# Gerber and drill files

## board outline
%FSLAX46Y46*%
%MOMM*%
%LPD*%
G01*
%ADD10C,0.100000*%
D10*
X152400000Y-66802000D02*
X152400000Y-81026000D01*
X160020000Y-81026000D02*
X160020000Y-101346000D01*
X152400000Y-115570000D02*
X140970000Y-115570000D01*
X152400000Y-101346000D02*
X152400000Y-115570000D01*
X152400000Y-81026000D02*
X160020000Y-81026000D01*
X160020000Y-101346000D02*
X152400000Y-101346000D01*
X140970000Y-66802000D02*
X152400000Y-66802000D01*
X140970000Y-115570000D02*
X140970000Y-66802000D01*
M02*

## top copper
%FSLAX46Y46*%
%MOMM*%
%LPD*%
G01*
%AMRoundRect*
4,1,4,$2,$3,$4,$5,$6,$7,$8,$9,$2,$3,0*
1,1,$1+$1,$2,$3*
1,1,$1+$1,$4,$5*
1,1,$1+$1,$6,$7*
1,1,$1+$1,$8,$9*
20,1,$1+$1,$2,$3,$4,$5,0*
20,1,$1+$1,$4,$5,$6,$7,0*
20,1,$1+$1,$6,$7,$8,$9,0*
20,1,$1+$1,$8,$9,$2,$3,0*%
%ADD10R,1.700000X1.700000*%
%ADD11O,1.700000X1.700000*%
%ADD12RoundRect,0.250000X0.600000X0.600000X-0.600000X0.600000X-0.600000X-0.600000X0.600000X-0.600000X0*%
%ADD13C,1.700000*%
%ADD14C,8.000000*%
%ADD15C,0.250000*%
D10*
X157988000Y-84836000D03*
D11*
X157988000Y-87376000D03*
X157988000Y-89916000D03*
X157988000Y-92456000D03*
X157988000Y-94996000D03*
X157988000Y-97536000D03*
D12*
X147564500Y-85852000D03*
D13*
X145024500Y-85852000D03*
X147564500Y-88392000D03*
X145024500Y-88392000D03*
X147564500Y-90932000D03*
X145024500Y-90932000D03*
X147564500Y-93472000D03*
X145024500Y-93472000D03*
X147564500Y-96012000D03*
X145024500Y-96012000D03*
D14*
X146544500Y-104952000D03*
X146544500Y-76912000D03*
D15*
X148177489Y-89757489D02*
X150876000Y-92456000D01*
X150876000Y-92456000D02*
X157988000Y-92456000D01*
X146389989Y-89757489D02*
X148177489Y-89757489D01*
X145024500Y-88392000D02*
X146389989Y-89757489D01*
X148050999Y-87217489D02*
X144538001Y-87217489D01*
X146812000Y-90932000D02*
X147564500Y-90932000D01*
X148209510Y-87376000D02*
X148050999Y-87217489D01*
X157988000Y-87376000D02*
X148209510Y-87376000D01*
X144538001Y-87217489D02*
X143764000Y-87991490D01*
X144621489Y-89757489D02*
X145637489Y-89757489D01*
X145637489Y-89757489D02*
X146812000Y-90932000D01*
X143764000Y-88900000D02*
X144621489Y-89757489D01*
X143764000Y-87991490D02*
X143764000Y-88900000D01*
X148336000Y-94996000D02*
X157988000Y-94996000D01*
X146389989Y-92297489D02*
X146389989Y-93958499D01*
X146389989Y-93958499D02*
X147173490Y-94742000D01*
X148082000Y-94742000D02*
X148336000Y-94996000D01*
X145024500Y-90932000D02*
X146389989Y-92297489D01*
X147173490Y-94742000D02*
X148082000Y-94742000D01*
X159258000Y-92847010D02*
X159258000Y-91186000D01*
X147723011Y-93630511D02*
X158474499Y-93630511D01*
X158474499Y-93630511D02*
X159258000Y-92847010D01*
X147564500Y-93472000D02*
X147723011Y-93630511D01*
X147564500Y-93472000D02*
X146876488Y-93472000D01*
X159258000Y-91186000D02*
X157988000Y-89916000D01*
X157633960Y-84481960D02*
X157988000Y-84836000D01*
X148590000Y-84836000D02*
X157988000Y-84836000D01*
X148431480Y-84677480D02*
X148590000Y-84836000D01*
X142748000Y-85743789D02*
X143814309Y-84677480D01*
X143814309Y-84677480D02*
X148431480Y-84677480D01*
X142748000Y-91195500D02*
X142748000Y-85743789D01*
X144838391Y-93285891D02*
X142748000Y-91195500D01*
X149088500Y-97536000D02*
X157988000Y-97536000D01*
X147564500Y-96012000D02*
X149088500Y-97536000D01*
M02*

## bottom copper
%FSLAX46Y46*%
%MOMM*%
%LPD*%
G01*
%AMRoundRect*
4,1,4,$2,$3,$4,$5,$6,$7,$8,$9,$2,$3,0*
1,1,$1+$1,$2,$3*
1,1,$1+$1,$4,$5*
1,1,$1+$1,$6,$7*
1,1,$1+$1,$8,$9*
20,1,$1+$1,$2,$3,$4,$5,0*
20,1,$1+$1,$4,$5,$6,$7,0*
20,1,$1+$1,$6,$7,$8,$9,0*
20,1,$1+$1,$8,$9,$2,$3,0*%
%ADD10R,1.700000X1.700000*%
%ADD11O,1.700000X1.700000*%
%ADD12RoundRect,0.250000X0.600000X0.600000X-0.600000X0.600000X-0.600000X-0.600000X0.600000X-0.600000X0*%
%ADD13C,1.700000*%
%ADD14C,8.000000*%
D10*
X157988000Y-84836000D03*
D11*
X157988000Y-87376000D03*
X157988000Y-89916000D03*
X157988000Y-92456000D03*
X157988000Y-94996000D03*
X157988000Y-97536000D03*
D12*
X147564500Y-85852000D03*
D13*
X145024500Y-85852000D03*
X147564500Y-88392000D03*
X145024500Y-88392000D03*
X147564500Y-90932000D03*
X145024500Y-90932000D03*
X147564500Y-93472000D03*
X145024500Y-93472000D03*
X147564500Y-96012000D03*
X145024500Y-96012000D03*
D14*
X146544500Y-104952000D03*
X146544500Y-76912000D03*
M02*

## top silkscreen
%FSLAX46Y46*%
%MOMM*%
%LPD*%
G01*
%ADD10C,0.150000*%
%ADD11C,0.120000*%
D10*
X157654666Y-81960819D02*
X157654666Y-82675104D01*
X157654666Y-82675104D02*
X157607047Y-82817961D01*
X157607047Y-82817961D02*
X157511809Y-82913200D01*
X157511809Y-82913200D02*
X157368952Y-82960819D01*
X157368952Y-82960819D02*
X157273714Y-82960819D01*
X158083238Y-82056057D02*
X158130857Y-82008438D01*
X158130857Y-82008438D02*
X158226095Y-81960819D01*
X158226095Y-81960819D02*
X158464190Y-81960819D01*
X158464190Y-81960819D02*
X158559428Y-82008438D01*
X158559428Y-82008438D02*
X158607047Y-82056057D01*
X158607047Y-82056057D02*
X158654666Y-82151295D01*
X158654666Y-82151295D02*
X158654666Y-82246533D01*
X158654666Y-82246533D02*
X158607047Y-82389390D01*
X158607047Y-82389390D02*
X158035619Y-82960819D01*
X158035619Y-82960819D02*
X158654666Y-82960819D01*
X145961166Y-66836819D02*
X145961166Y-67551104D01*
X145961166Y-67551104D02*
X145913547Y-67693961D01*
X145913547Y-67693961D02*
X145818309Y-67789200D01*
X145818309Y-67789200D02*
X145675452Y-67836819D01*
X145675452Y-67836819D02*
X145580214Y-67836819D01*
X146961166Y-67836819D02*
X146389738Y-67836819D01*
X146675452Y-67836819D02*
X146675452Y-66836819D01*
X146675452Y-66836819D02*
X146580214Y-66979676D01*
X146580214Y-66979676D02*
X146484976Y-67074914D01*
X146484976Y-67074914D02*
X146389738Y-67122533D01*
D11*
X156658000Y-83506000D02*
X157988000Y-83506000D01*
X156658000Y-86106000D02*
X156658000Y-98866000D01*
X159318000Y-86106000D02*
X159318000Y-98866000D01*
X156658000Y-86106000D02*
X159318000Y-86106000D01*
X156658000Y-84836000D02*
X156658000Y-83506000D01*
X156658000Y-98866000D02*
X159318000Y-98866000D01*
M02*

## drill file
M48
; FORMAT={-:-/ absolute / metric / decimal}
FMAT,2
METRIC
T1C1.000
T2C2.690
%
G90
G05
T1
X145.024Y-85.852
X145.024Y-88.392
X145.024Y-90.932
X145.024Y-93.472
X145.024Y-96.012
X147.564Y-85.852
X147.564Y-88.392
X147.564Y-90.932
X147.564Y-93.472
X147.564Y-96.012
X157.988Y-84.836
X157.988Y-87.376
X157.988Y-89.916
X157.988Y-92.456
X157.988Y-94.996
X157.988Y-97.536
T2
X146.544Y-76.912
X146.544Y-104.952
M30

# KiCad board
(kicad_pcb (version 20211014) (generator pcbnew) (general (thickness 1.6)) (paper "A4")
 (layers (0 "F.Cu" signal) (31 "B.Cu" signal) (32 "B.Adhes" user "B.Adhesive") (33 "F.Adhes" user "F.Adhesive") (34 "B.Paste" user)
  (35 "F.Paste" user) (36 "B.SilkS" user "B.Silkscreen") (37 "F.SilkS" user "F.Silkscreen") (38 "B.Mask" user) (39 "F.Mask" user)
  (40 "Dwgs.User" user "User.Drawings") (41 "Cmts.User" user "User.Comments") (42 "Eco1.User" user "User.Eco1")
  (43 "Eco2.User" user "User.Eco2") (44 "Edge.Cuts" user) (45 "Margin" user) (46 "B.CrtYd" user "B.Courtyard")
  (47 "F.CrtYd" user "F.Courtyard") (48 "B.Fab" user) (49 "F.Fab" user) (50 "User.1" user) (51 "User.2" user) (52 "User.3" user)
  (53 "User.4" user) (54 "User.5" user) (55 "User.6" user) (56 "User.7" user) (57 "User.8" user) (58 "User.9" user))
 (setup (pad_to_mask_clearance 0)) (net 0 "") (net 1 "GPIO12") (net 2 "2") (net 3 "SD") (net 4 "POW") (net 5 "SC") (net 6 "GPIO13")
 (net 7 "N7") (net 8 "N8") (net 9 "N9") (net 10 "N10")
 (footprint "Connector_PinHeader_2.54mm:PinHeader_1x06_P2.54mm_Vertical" (layer "F.Cu") (at 157.988 84.836)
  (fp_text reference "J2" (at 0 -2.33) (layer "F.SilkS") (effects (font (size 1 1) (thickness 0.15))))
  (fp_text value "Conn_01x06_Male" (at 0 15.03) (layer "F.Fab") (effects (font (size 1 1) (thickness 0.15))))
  (fp_line (start -1.33 -1.33) (end 0 -1.33) (layer "F.SilkS") (width 0.12))
  (fp_line (start -1.33 1.27) (end -1.33 14.03) (layer "F.SilkS") (width 0.12))
  (fp_line (start 1.33 1.27) (end 1.33 14.03) (layer "F.SilkS") (width 0.12))
  (fp_line (start -1.33 1.27) (end 1.33 1.27) (layer "F.SilkS") (width 0.12))
  (fp_line (start -1.33 0) (end -1.33 -1.33) (layer "F.SilkS") (width 0.12))
  (fp_line (start -1.33 14.03) (end 1.33 14.03) (layer "F.SilkS") (width 0.12))
  (pad "1" thru_hole rect (at 0 0) (size 1.7 1.7) (drill 1) (layers *.Cu *.Mask) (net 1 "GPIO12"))
  (pad "2" thru_hole oval (at 0 2.54) (size 1.7 1.7) (drill 1) (layers *.Cu *.Mask) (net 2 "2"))
  (pad "3" thru_hole oval (at 0 5.08) (size 1.7 1.7) (drill 1) (layers *.Cu *.Mask) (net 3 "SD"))
  (pad "4" thru_hole oval (at 0 7.62) (size 1.7 1.7) (drill 1) (layers *.Cu *.Mask) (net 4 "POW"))
  (pad "5" thru_hole oval (at 0 10.16) (size 1.7 1.7) (drill 1) (layers *.Cu *.Mask) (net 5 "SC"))
  (pad "6" thru_hole oval (at 0 12.7) (size 1.7 1.7) (drill 1) (layers *.Cu *.Mask) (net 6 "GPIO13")))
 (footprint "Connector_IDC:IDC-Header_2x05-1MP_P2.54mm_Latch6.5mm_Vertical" (layer "B.Cu") (at 147.5645 85.852 180)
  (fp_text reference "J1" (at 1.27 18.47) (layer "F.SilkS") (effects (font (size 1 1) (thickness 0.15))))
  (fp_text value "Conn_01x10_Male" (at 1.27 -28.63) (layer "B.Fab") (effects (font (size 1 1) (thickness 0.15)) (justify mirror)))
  (pad "1" thru_hole roundrect (at 0 0 180) (size 1.7 1.7) (drill 1) (layers *.Cu *.Mask) (roundrect_rratio 0.147059) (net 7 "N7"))
  (pad "2" thru_hole circle (at 2.54 0 180) (size 1.7 1.7) (drill 1) (layers *.Cu *.Mask) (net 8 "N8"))
  (pad "3" thru_hole circle (at 0 -2.54 180) (size 1.7 1.7) (drill 1) (layers *.Cu *.Mask) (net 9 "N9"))
  (pad "4" thru_hole circle (at 2.54 -2.54 180) (size 1.7 1.7) (drill 1) (layers *.Cu *.Mask) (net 4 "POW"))
  (pad "5" thru_hole circle (at 0 -5.08 180) (size 1.7 1.7) (drill 1) (layers *.Cu *.Mask) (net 2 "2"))
  (pad "6" thru_hole circle (at 2.54 -5.08 180) (size 1.7 1.7) (drill 1) (layers *.Cu *.Mask) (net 5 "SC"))
  (pad "7" thru_hole circle (at 0 -7.62 180) (size 1.7 1.7) (drill 1) (layers *.Cu *.Mask) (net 3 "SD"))
  (pad "8" thru_hole circle (at 2.54 -7.62 180) (size 1.7 1.7) (drill 1) (layers *.Cu *.Mask) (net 1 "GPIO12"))
  (pad "9" thru_hole circle (at 0 -10.16 180) (size 1.7 1.7) (drill 1) (layers *.Cu *.Mask) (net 6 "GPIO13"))
  (pad "10" thru_hole circle (at 2.54 -10.16 180) (size 1.7 1.7) (drill 1) (layers *.Cu *.Mask) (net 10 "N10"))
  (pad "MP" thru_hole circle (at 1.02 -19.1 180) (size 8 8) (drill 2.69) (layers *.Cu *.Mask))
  (pad "MP" thru_hole circle (at 1.02 8.94 180) (size 8 8) (drill 2.69) (layers *.Cu *.Mask)))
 (gr_line (start 152.4 66.802) (end 152.4 81.026) (layer "Edge.Cuts") (width 0.1))
 (gr_line (start 160.02 81.026) (end 160.02 101.346) (layer "Edge.Cuts") (width 0.1))
 (gr_line (start 152.4 115.57) (end 140.97 115.57) (layer "Edge.Cuts") (width 0.1))
 (gr_line (start 152.4 101.346) (end 152.4 115.57) (layer "Edge.Cuts") (width 0.1))
 (gr_line (start 152.4 81.026) (end 160.02 81.026) (layer "Edge.Cuts") (width 0.1))
 (gr_line (start 160.02 101.346) (end 152.4 101.346) (layer "Edge.Cuts") (width 0.1))
 (gr_line (start 140.97 66.802) (end 152.4 66.802) (layer "Edge.Cuts") (width 0.1))
 (gr_line (start 140.97 115.57) (end 140.97 66.802) (layer "Edge.Cuts") (width 0.1))
 (segment (start 148.177489 89.757489) (end 150.876 92.456) (width 0.25) (layer "F.Cu") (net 4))
 (segment (start 150.876 92.456) (end 157.988 92.456) (width 0.25) (layer "F.Cu") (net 4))
 (segment (start 146.389989 89.757489) (end 148.177489 89.757489) (width 0.25) (layer "F.Cu") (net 4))
 (segment (start 145.0245 88.392) (end 146.389989 89.757489) (width 0.25) (layer "F.Cu") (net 4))
 (segment (start 148.050999 87.217489) (end 144.538001 87.217489) (width 0.25) (layer "F.Cu") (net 2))
 (segment (start 146.812 90.932) (end 147.5645 90.932) (width 0.25) (layer "F.Cu") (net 2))
 (segment (start 148.20951 87.376) (end 148.050999 87.217489) (width 0.25) (layer "F.Cu") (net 2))
 (segment (start 157.988 87.376) (end 148.20951 87.376) (width 0.25) (layer "F.Cu") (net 2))
 (segment (start 144.538001 87.217489) (end 143.764 87.99149) (width 0.25) (layer "F.Cu") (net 2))
 (segment (start 144.621489 89.757489) (end 145.637489 89.757489) (width 0.25) (layer "F.Cu") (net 2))
 (segment (start 145.637489 89.757489) (end 146.812 90.932) (width 0.25) (layer "F.Cu") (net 2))
 (segment (start 143.764 88.9) (end 144.621489 89.757489) (width 0.25) (layer "F.Cu") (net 2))
 (segment (start 143.764 87.99149) (end 143.764 88.9) (width 0.25) (layer "F.Cu") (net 2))
 (segment (start 148.336 94.996) (end 157.988 94.996) (width 0.25) (layer "F.Cu") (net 5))
 (segment (start 146.389989 92.297489) (end 146.389989 93.958499) (width 0.25) (layer "F.Cu") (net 5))
 (segment (start 146.389989 93.958499) (end 147.17349 94.742) (width 0.25) (layer "F.Cu") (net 5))
 (segment (start 148.082 94.742) (end 148.336 94.996) (width 0.25) (layer "F.Cu") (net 5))
 (segment (start 145.0245 90.932) (end 146.389989 92.297489) (width 0.25) (layer "F.Cu") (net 5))
 (segment (start 147.17349 94.742) (end 148.082 94.742) (width 0.25) (layer "F.Cu") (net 5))
 (segment (start 159.258 92.84701) (end 159.258 91.186) (width 0.25) (layer "F.Cu") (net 3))
 (segment (start 147.723011 93.630511) (end 158.474499 93.630511) (width 0.25) (layer "F.Cu") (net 3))
 (segment (start 158.474499 93.630511) (end 159.258 92.84701) (width 0.25) (layer "F.Cu") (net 3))
 (segment (start 147.5645 93.472) (end 147.723011 93.630511) (width 0.25) (layer "F.Cu") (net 3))
 (segment (start 147.5645 93.472) (end 146.876488 93.472) (width 0.25) (layer "F.Cu") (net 3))
 (segment (start 159.258 91.186) (end 157.988 89.916) (width 0.25) (layer "F.Cu") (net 3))
 (segment (start 157.63396 84.48196) (end 157.988 84.836) (width 0.25) (layer "F.Cu") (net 1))
 (segment (start 148.59 84.836) (end 157.988 84.836) (width 0.25) (layer "F.Cu") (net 1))
 (segment (start 148.43148 84.67748) (end 148.59 84.836) (width 0.25) (layer "F.Cu") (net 1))
 (segment (start 142.748 85.743789) (end 143.814309 84.67748) (width 0.25) (layer "F.Cu") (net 1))
 (segment (start 143.814309 84.67748) (end 148.43148 84.67748) (width 0.25) (layer "F.Cu") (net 1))
 (segment (start 142.748 91.1955) (end 142.748 85.743789) (width 0.25) (layer "F.Cu") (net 1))
 (segment (start 144.838391 93.285891) (end 142.748 91.1955) (width 0.25) (layer "F.Cu") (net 1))
 (segment (start 149.0885 97.536) (end 157.988 97.536) (width 0.25) (layer "F.Cu") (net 6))
 (segment (start 147.5645 96.012) (end 149.0885 97.536) (width 0.25) (layer "F.Cu") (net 6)))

